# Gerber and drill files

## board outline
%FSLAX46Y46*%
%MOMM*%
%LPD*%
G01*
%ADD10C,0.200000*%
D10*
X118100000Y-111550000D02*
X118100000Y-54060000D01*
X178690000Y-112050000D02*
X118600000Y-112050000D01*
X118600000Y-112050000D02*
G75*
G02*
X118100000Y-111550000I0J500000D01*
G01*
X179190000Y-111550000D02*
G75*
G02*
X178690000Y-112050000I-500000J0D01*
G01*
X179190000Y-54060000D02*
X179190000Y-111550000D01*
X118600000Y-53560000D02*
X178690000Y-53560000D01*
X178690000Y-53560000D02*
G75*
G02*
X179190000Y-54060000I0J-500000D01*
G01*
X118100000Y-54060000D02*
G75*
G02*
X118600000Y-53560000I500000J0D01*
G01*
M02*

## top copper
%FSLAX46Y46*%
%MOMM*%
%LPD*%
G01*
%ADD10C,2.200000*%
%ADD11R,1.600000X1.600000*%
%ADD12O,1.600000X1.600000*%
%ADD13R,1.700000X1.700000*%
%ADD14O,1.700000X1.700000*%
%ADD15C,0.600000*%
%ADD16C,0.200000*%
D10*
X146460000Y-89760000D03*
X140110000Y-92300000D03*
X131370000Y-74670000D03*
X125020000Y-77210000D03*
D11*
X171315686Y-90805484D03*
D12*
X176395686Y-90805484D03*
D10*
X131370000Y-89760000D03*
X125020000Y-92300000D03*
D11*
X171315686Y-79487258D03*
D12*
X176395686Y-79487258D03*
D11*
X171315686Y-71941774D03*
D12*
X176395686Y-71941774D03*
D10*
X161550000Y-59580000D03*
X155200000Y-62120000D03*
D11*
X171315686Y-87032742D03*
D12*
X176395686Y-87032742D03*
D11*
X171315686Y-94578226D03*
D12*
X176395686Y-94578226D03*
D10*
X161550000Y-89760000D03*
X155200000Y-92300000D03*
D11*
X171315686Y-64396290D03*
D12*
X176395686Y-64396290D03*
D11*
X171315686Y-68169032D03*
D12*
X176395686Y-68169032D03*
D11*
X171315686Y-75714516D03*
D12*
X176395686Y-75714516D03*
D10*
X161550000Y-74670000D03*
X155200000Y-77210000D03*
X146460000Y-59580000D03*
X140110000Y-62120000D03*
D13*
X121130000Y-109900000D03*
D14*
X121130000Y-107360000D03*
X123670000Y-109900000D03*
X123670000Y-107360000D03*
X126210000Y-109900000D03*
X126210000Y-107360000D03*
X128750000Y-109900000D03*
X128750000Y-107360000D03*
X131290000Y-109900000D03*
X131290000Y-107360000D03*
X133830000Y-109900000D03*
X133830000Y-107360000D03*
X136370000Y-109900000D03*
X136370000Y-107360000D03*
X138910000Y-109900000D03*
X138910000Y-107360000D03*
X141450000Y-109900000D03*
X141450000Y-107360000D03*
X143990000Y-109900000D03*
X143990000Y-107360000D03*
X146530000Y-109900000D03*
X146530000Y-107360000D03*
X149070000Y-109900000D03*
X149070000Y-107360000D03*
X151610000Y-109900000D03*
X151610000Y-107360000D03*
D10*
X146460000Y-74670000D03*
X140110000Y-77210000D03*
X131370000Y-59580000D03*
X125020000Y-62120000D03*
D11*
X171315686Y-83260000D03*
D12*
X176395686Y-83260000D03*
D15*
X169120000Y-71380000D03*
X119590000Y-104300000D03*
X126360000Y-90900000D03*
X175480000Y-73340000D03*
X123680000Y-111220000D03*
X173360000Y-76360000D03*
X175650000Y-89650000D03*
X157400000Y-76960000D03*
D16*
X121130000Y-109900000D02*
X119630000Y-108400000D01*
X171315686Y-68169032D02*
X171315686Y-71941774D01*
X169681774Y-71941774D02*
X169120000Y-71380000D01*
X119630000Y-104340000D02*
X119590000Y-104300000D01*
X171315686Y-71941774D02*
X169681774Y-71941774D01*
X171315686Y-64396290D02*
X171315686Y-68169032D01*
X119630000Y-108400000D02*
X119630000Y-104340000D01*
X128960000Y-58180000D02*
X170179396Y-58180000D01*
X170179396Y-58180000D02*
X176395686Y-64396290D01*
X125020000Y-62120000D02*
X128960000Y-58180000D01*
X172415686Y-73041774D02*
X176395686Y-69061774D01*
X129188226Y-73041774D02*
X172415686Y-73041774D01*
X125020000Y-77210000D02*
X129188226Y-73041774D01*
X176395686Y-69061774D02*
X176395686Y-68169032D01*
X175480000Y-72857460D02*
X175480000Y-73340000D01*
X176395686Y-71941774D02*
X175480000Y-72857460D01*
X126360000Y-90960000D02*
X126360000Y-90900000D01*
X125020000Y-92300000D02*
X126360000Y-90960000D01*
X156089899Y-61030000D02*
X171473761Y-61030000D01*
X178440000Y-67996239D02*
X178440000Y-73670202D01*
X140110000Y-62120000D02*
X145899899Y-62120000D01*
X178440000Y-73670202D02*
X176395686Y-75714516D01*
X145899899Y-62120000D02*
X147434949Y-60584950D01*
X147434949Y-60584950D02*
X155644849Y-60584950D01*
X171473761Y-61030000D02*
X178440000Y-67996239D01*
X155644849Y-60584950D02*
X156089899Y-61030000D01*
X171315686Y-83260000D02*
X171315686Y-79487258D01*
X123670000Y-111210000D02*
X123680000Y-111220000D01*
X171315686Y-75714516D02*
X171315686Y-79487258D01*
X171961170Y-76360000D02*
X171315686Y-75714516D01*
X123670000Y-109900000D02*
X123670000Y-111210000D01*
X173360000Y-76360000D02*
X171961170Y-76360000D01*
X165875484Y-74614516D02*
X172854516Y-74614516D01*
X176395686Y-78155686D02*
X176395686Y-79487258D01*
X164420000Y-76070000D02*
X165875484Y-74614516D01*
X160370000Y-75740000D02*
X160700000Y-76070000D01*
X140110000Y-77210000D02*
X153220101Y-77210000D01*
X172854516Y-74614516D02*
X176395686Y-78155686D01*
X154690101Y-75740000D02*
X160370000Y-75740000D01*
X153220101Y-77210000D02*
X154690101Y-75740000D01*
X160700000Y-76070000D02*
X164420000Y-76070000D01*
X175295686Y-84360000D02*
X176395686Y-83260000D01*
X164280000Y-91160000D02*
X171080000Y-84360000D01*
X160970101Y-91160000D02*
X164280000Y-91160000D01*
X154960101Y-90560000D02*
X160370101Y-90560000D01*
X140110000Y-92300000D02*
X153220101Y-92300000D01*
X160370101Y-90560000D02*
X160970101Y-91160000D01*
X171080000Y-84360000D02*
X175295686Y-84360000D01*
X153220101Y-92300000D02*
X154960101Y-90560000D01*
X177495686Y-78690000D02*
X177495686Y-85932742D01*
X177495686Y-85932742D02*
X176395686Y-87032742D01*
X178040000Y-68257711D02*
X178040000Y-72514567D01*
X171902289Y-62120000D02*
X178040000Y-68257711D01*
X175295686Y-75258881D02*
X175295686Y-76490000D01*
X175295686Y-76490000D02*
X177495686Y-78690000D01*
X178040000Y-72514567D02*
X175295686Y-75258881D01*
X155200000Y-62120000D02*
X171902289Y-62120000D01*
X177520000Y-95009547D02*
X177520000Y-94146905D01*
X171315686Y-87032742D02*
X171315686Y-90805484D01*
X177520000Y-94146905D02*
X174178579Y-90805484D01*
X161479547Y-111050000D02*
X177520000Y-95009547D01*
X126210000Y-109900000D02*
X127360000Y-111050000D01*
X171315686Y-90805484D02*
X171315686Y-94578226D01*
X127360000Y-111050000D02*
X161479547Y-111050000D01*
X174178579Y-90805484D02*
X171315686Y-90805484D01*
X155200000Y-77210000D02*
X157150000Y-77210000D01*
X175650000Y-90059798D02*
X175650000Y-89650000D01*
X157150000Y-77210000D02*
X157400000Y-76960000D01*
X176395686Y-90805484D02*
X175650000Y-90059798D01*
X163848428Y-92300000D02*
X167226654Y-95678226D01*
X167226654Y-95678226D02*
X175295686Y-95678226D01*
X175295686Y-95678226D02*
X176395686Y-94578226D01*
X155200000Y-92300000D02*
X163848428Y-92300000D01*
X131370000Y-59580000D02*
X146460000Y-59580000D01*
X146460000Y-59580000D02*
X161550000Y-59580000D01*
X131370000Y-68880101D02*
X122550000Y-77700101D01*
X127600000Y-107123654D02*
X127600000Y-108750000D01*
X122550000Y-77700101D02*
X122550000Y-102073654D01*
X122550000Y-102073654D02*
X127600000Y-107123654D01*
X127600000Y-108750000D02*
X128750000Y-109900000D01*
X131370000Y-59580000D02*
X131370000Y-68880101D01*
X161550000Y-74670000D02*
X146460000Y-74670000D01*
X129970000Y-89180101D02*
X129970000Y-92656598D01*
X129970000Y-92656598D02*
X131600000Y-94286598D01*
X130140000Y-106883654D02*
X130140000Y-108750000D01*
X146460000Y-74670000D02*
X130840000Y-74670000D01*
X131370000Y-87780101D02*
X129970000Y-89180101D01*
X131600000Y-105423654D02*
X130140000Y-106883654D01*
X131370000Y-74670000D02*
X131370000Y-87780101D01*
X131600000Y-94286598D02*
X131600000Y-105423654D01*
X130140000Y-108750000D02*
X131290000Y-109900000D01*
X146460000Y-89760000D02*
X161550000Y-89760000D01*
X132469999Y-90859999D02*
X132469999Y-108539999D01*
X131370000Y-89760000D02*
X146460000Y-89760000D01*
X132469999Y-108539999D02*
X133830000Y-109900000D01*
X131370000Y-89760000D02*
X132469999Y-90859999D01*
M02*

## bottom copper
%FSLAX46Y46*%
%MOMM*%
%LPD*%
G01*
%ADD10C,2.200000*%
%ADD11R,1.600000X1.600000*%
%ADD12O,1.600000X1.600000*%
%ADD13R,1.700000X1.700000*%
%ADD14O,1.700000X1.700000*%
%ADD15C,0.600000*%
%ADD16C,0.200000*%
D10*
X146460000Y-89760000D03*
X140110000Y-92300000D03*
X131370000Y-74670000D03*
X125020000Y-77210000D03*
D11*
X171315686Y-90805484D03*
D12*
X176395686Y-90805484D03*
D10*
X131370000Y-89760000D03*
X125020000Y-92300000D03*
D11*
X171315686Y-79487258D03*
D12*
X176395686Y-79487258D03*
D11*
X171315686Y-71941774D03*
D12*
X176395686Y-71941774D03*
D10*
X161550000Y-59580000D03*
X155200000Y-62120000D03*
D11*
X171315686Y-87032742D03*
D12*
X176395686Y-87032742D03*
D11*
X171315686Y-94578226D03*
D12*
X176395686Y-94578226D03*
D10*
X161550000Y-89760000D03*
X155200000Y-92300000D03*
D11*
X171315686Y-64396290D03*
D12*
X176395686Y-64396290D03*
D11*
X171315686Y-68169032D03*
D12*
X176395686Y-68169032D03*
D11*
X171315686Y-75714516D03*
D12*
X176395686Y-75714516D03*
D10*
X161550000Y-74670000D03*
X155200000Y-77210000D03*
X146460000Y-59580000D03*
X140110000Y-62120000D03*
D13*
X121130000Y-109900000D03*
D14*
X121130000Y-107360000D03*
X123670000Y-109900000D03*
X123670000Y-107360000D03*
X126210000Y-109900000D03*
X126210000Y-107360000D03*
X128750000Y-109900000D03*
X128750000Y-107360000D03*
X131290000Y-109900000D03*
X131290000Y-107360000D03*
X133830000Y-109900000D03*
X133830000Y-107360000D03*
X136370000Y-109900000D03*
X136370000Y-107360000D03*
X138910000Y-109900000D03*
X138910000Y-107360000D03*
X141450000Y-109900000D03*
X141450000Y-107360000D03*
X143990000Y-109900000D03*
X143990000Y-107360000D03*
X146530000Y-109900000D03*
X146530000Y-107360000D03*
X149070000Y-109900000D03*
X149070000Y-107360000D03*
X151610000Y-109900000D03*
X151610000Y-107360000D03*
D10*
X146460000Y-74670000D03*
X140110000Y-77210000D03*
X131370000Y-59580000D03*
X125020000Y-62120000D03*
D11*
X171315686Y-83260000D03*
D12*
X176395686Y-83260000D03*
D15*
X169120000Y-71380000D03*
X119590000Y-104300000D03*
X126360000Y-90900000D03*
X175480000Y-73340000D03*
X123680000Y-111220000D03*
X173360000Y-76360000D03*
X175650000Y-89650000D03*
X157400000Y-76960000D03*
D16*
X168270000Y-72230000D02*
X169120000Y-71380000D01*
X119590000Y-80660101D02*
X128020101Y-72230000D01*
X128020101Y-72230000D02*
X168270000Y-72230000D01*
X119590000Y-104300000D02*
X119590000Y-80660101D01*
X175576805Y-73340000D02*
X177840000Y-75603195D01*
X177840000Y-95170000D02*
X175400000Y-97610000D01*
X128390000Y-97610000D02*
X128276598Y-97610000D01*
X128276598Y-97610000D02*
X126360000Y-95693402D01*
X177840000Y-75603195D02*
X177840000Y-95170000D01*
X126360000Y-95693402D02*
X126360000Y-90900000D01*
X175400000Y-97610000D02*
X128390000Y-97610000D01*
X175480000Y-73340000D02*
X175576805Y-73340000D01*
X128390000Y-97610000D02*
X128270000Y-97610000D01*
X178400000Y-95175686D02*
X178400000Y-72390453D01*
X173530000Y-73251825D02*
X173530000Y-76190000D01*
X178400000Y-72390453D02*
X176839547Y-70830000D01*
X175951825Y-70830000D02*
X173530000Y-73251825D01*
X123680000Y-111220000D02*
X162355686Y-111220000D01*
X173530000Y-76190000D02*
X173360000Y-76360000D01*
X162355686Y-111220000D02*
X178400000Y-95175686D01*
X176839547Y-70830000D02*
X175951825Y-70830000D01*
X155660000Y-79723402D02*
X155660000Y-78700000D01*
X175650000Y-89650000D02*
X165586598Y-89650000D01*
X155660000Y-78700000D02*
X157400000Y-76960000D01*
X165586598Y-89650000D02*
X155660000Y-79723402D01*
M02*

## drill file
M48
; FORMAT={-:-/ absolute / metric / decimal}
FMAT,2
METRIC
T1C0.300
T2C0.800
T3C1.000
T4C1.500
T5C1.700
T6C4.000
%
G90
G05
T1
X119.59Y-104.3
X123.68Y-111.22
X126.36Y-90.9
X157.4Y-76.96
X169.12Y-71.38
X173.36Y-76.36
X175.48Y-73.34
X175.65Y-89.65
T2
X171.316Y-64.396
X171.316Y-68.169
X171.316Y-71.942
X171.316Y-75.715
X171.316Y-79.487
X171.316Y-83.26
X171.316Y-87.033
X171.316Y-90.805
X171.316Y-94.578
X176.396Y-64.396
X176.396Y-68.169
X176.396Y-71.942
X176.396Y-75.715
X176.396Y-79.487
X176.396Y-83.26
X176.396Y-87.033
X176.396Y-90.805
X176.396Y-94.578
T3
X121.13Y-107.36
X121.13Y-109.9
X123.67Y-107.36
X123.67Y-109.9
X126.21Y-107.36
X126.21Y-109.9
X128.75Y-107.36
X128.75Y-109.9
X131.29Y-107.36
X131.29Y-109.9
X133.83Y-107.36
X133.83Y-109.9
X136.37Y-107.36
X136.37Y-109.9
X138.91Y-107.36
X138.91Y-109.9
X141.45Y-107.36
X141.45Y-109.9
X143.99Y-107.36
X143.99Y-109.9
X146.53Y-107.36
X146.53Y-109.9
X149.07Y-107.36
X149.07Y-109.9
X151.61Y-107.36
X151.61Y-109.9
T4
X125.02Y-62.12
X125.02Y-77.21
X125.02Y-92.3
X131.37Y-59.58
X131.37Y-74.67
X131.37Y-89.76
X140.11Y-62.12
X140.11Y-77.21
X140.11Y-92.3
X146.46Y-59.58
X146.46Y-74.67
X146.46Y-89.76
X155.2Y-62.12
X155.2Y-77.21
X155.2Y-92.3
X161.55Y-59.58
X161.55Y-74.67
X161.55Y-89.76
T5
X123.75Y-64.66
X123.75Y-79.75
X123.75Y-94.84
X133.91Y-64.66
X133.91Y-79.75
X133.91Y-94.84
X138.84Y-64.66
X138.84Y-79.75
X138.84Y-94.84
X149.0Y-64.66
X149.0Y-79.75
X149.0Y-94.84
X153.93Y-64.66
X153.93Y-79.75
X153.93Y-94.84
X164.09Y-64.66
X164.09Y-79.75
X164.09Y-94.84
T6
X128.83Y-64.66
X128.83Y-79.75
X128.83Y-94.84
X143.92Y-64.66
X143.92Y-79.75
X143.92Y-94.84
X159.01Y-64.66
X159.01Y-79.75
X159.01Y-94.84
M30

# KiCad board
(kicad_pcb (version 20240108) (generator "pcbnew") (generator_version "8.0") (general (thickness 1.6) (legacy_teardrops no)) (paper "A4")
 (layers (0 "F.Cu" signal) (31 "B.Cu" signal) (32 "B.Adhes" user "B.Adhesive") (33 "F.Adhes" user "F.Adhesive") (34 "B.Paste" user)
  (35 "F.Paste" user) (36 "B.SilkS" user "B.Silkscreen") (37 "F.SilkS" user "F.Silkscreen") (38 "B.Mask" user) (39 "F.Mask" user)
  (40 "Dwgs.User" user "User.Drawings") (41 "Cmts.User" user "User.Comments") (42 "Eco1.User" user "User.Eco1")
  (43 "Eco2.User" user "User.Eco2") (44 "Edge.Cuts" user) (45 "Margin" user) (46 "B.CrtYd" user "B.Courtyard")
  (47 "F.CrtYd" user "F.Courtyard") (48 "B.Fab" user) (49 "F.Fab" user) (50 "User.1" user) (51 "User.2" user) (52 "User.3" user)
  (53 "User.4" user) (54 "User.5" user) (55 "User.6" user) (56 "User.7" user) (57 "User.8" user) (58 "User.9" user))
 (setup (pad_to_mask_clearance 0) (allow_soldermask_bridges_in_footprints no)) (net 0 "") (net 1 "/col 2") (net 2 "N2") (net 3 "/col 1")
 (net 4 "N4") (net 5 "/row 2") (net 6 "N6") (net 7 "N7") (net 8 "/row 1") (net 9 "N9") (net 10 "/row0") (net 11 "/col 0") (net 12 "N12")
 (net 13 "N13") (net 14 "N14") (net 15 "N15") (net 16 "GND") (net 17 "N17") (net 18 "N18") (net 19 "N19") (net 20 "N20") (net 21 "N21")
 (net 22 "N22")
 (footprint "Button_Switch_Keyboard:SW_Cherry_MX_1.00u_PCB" (layer "F.Cu") (at 146.46 89.76)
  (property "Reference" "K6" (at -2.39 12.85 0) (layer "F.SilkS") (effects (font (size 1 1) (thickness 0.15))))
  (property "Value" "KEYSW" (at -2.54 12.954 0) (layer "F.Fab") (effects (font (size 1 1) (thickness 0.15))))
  (pad "" np_thru_hole circle (at -7.62 5.08) (size 1.7 1.7) (drill 1.7) (layers "*.Cu" "*.Mask"))
  (pad "" np_thru_hole circle (at -2.54 5.08) (size 4 4) (drill 4) (layers "*.Cu" "*.Mask"))
  (pad "" np_thru_hole circle (at 2.54 5.08) (size 1.7 1.7) (drill 1.7) (layers "*.Cu" "*.Mask"))
  (pad "1" thru_hole circle (at 0 0) (size 2.2 2.2) (drill 1.5) (layers "*.Cu" "*.Mask") (remove_unused_layers no) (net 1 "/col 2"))
  (pad "2" thru_hole circle (at -6.35 2.54) (size 2.2 2.2) (drill 1.5) (layers "*.Cu" "*.Mask") (remove_unused_layers no) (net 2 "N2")))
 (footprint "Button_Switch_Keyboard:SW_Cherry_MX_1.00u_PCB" (layer "F.Cu") (at 131.37 74.67)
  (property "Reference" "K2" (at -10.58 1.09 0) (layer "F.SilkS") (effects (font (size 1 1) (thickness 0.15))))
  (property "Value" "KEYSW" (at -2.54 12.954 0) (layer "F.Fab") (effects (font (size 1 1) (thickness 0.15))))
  (pad "" np_thru_hole circle (at -7.62 5.08) (size 1.7 1.7) (drill 1.7) (layers "*.Cu" "*.Mask"))
  (pad "" np_thru_hole circle (at -2.54 5.08) (size 4 4) (drill 4) (layers "*.Cu" "*.Mask"))
  (pad "" np_thru_hole circle (at 2.54 5.08) (size 1.7 1.7) (drill 1.7) (layers "*.Cu" "*.Mask"))
  (pad "1" thru_hole circle (at 0 0) (size 2.2 2.2) (drill 1.5) (layers "*.Cu" "*.Mask") (remove_unused_layers no) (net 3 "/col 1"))
  (pad "2" thru_hole circle (at -6.35 2.54) (size 2.2 2.2) (drill 1.5) (layers "*.Cu" "*.Mask") (remove_unused_layers no) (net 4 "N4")))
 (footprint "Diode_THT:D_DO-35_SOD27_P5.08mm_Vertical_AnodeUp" (layer "F.Cu") (at 171.315686 90.805484)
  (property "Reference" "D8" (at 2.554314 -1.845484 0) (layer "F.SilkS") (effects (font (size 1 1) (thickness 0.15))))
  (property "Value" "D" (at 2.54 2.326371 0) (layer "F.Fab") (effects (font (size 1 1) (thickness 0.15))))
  (pad "1" thru_hole rect (at 0 0) (size 1.6 1.6) (drill 0.8) (layers "*.Cu" "*.Mask") (remove_unused_layers no) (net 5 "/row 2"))
  (pad "2" thru_hole oval (at 5.08 0) (size 1.6 1.6) (drill 0.8) (layers "*.Cu" "*.Mask") (remove_unused_layers no) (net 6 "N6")))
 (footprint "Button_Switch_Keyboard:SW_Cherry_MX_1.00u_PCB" (layer "F.Cu") (at 131.37 89.76)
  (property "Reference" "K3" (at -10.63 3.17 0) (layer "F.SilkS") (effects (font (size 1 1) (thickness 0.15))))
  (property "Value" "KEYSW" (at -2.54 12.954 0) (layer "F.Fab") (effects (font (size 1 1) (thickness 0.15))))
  (pad "" np_thru_hole circle (at -7.62 5.08) (size 1.7 1.7) (drill 1.7) (layers "*.Cu" "*.Mask"))
  (pad "" np_thru_hole circle (at -2.54 5.08) (size 4 4) (drill 4) (layers "*.Cu" "*.Mask"))
  (pad "" np_thru_hole circle (at 2.54 5.08) (size 1.7 1.7) (drill 1.7) (layers "*.Cu" "*.Mask"))
  (pad "1" thru_hole circle (at 0 0) (size 2.2 2.2) (drill 1.5) (layers "*.Cu" "*.Mask") (remove_unused_layers no) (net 1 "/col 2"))
  (pad "2" thru_hole circle (at -6.35 2.54) (size 2.2 2.2) (drill 1.5) (layers "*.Cu" "*.Mask") (remove_unused_layers no) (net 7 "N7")))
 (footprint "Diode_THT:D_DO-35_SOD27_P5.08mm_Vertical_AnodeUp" (layer "F.Cu") (at 171.315686 79.487258)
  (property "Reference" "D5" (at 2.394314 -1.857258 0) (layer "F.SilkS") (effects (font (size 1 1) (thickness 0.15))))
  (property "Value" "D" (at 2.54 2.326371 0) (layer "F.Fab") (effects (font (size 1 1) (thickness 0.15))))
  (pad "1" thru_hole rect (at 0 0) (size 1.6 1.6) (drill 0.8) (layers "*.Cu" "*.Mask") (remove_unused_layers no) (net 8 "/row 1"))
  (pad "2" thru_hole oval (at 5.08 0) (size 1.6 1.6) (drill 0.8) (layers "*.Cu" "*.Mask") (remove_unused_layers no) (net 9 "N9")))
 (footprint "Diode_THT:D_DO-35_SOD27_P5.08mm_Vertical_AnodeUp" (layer "F.Cu") (at 171.315686 71.941774)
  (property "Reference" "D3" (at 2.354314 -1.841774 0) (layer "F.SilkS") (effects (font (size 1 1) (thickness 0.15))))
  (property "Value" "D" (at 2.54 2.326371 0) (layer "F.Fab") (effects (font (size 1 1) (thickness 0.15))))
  (pad "1" thru_hole rect (at 0 0) (size 1.6 1.6) (drill 0.8) (layers "*.Cu" "*.Mask") (remove_unused_layers no) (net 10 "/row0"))
  (pad "2" thru_hole oval (at 5.08 0) (size 1.6 1.6) (drill 0.8) (layers "*.Cu" "*.Mask") (remove_unused_layers no) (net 7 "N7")))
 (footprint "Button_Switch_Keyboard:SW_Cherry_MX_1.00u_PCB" (layer "F.Cu") (at 161.55 59.58)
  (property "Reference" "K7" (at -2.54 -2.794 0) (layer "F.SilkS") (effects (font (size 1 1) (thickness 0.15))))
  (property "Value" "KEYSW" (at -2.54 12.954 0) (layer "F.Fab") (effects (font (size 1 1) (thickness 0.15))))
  (pad "" np_thru_hole circle (at -7.62 5.08) (size 1.7 1.7) (drill 1.7) (layers "*.Cu" "*.Mask"))
  (pad "" np_thru_hole circle (at -2.54 5.08) (size 4 4) (drill 4) (layers "*.Cu" "*.Mask"))
  (pad "" np_thru_hole circle (at 2.54 5.08) (size 1.7 1.7) (drill 1.7) (layers "*.Cu" "*.Mask"))
  (pad "1" thru_hole circle (at 0 0) (size 2.2 2.2) (drill 1.5) (layers "*.Cu" "*.Mask") (remove_unused_layers no) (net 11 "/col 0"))
  (pad "2" thru_hole circle (at -6.35 2.54) (size 2.2 2.2) (drill 1.5) (layers "*.Cu" "*.Mask") (remove_unused_layers no) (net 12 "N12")))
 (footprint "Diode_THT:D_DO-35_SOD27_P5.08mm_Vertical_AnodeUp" (layer "F.Cu") (at 171.315686 87.032742)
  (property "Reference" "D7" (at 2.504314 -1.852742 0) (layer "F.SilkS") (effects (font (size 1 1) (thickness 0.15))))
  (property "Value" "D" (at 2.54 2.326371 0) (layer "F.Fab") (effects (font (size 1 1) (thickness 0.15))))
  (pad "1" thru_hole rect (at 0 0) (size 1.6 1.6) (drill 0.8) (layers "*.Cu" "*.Mask") (remove_unused_layers no) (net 5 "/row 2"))
  (pad "2" thru_hole oval (at 5.08 0) (size 1.6 1.6) (drill 0.8) (layers "*.Cu" "*.Mask") (remove_unused_layers no) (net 12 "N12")))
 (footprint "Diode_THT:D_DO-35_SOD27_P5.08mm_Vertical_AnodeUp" (layer "F.Cu") (at 171.315686 94.578226)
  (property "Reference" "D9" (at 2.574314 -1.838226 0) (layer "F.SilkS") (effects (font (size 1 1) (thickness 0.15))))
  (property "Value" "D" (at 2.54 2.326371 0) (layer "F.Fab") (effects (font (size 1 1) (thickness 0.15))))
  (pad "1" thru_hole rect (at 0 0) (size 1.6 1.6) (drill 0.8) (layers "*.Cu" "*.Mask") (remove_unused_layers no) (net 5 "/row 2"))
  (pad "2" thru_hole oval (at 5.08 0) (size 1.6 1.6) (drill 0.8) (layers "*.Cu" "*.Mask") (remove_unused_layers no) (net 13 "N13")))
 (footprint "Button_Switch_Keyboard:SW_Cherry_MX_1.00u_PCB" (layer "F.Cu") (at 161.55 89.76)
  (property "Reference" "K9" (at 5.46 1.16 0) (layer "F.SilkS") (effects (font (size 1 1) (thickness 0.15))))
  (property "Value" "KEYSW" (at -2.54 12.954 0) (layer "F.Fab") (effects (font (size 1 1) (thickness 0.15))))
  (pad "" np_thru_hole circle (at -7.62 5.08) (size 1.7 1.7) (drill 1.7) (layers "*.Cu" "*.Mask"))
  (pad "" np_thru_hole circle (at -2.54 5.08) (size 4 4) (drill 4) (layers "*.Cu" "*.Mask"))
  (pad "" np_thru_hole circle (at 2.54 5.08) (size 1.7 1.7) (drill 1.7) (layers "*.Cu" "*.Mask"))
  (pad "1" thru_hole circle (at 0 0) (size 2.2 2.2) (drill 1.5) (layers "*.Cu" "*.Mask") (remove_unused_layers no) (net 1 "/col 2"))
  (pad "2" thru_hole circle (at -6.35 2.54) (size 2.2 2.2) (drill 1.5) (layers "*.Cu" "*.Mask") (remove_unused_layers no) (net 13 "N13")))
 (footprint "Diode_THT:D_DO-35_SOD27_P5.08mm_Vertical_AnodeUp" (layer "F.Cu") (at 171.315686 64.39629)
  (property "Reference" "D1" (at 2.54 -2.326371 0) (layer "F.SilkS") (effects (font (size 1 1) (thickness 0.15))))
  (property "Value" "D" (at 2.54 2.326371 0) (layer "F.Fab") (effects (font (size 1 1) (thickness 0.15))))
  (pad "1" thru_hole rect (at 0 0) (size 1.6 1.6) (drill 0.8) (layers "*.Cu" "*.Mask") (remove_unused_layers no) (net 10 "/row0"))
  (pad "2" thru_hole oval (at 5.08 0) (size 1.6 1.6) (drill 0.8) (layers "*.Cu" "*.Mask") (remove_unused_layers no) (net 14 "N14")))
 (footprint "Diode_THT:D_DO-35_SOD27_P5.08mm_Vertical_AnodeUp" (layer "F.Cu") (at 171.315686 68.169032)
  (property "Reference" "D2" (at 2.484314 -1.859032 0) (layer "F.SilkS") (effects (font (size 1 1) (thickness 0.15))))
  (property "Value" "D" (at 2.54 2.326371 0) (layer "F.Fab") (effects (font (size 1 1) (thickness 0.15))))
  (pad "1" thru_hole rect (at 0 0) (size 1.6 1.6) (drill 0.8) (layers "*.Cu" "*.Mask") (remove_unused_layers no) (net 10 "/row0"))
  (pad "2" thru_hole oval (at 5.08 0) (size 1.6 1.6) (drill 0.8) (layers "*.Cu" "*.Mask") (remove_unused_layers no) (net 4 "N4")))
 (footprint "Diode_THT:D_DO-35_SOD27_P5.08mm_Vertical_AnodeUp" (layer "F.Cu") (at 171.315686 75.714516)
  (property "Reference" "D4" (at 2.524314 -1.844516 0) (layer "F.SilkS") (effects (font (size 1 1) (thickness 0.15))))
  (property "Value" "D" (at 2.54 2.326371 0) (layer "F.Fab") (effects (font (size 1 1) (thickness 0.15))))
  (pad "1" thru_hole rect (at 0 0) (size 1.6 1.6) (drill 0.8) (layers "*.Cu" "*.Mask") (remove_unused_layers no) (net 8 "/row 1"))
  (pad "2" thru_hole oval (at 5.08 0) (size 1.6 1.6) (drill 0.8) (layers "*.Cu" "*.Mask") (remove_unused_layers no) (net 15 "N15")))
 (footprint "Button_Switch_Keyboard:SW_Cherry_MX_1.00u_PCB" (layer "F.Cu") (at 161.55 74.67)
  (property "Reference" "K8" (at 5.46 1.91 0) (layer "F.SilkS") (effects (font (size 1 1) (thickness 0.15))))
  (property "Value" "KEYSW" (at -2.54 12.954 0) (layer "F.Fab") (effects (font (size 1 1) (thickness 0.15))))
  (pad "" np_thru_hole circle (at -7.62 5.08) (size 1.7 1.7) (drill 1.7) (layers "*.Cu" "*.Mask"))
  (pad "" np_thru_hole circle (at -2.54 5.08) (size 4 4) (drill 4) (layers "*.Cu" "*.Mask"))
  (pad "" np_thru_hole circle (at 2.54 5.08) (size 1.7 1.7) (drill 1.7) (layers "*.Cu" "*.Mask"))
  (pad "1" thru_hole circle (at 0 0) (size 2.2 2.2) (drill 1.5) (layers "*.Cu" "*.Mask") (remove_unused_layers no) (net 3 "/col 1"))
  (pad "2" thru_hole circle (at -6.35 2.54) (size 2.2 2.2) (drill 1.5) (layers "*.Cu" "*.Mask") (remove_unused_layers no) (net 6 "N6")))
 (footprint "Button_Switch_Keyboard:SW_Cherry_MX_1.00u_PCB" (layer "F.Cu") (at 146.46 59.58)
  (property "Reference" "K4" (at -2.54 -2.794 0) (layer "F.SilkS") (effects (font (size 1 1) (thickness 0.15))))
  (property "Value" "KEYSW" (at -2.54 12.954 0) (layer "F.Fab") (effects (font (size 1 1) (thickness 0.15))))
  (pad "" np_thru_hole circle (at -7.62 5.08) (size 1.7 1.7) (drill 1.7) (layers "*.Cu" "*.Mask"))
  (pad "" np_thru_hole circle (at -2.54 5.08) (size 4 4) (drill 4) (layers "*.Cu" "*.Mask"))
  (pad "" np_thru_hole circle (at 2.54 5.08) (size 1.7 1.7) (drill 1.7) (layers "*.Cu" "*.Mask"))
  (pad "1" thru_hole circle (at 0 0) (size 2.2 2.2) (drill 1.5) (layers "*.Cu" "*.Mask") (remove_unused_layers no) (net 11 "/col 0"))
  (pad "2" thru_hole circle (at -6.35 2.54) (size 2.2 2.2) (drill 1.5) (layers "*.Cu" "*.Mask") (remove_unused_layers no) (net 15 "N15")))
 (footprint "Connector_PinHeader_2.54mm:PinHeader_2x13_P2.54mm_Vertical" (layer "F.Cu") (at 121.13 109.9 90)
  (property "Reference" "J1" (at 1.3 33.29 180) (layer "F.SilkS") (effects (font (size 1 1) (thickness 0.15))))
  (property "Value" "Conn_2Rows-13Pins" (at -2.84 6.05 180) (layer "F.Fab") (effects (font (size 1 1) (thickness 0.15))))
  (pad "1" thru_hole rect (at 0 0 90) (size 1.7 1.7) (drill 1) (layers "*.Cu" "*.Mask") (remove_unused_layers no) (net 10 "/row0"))
  (pad "2" thru_hole oval (at 2.54 0 90) (size 1.7 1.7) (drill 1) (layers "*.Cu" "*.Mask") (remove_unused_layers no) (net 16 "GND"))
  (pad "3" thru_hole oval (at 0 2.54 90) (size 1.7 1.7) (drill 1) (layers "*.Cu" "*.Mask") (remove_unused_layers no) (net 8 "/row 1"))
  (pad "4" thru_hole oval (at 2.54 2.54 90) (size 1.7 1.7) (drill 1) (layers "*.Cu" "*.Mask") (remove_unused_layers no) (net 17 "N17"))
  (pad "5" thru_hole oval (at 0 5.08 90) (size 1.7 1.7) (drill 1) (layers "*.Cu" "*.Mask") (remove_unused_layers no) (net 5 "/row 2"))
  (pad "6" thru_hole oval (at 2.54 5.08 90) (size 1.7 1.7) (drill 1) (layers "*.Cu" "*.Mask") (remove_unused_layers no) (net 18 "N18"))
  (pad "7" thru_hole oval (at 0 7.62 90) (size 1.7 1.7) (drill 1) (layers "*.Cu" "*.Mask") (remove_unused_layers no) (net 11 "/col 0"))
  (pad "8" thru_hole oval (at 2.54 7.62 90) (size 1.7 1.7) (drill 1) (layers "*.Cu" "*.Mask") (remove_unused_layers no) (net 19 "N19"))
  (pad "9" thru_hole oval (at 0 10.16 90) (size 1.7 1.7) (drill 1) (layers "*.Cu" "*.Mask") (remove_unused_layers no) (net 3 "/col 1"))
  (pad "10" thru_hole oval (at 2.54 10.16 90) (size 1.7 1.7) (drill 1) (layers "*.Cu" "*.Mask") (remove_unused_layers no) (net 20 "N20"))
  (pad "11" thru_hole oval (at 0 12.7 90) (size 1.7 1.7) (drill 1) (layers "*.Cu" "*.Mask") (remove_unused_layers no) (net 1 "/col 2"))
  (pad "12" thru_hole oval (at 2.54 12.7 90) (size 1.7 1.7) (drill 1) (layers "*.Cu" "*.Mask") (remove_unused_layers no) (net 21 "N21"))
  (pad "13" thru_hole oval (at 0 15.24 90) (size 1.7 1.7) (drill 1) (layers "*.Cu" "*.Mask") (remove_unused_layers no) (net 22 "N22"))
  (pad "14" thru_hole oval (at 2.54 15.24 90) (size 1.7 1.7) (drill 1) (layers "*.Cu" "*.Mask") (remove_unused_layers no))
  (pad "15" thru_hole oval (at 0 17.78 90) (size 1.7 1.7) (drill 1) (layers "*.Cu" "*.Mask") (remove_unused_layers no))
  (pad "16" thru_hole oval (at 2.54 17.78 90) (size 1.7 1.7) (drill 1) (layers "*.Cu" "*.Mask") (remove_unused_layers no))
  (pad "17" thru_hole oval (at 0 20.32 90) (size 1.7 1.7) (drill 1) (layers "*.Cu" "*.Mask") (remove_unused_layers no))
  (pad "18" thru_hole oval (at 2.54 20.32 90) (size 1.7 1.7) (drill 1) (layers "*.Cu" "*.Mask") (remove_unused_layers no))
  (pad "19" thru_hole oval (at 0 22.86 90) (size 1.7 1.7) (drill 1) (layers "*.Cu" "*.Mask") (remove_unused_layers no))
  (pad "20" thru_hole oval (at 2.54 22.86 90) (size 1.7 1.7) (drill 1) (layers "*.Cu" "*.Mask") (remove_unused_layers no))
  (pad "21" thru_hole oval (at 0 25.4 90) (size 1.7 1.7) (drill 1) (layers "*.Cu" "*.Mask") (remove_unused_layers no))
  (pad "22" thru_hole oval (at 2.54 25.4 90) (size 1.7 1.7) (drill 1) (layers "*.Cu" "*.Mask") (remove_unused_layers no))
  (pad "23" thru_hole oval (at 0 27.94 90) (size 1.7 1.7) (drill 1) (layers "*.Cu" "*.Mask") (remove_unused_layers no))
  (pad "24" thru_hole oval (at 2.54 27.94 90) (size 1.7 1.7) (drill 1) (layers "*.Cu" "*.Mask") (remove_unused_layers no))
  (pad "25" thru_hole oval (at 0 30.48 90) (size 1.7 1.7) (drill 1) (layers "*.Cu" "*.Mask") (remove_unused_layers no))
  (pad "26" thru_hole oval (at 2.54 30.48 90) (size 1.7 1.7) (drill 1) (layers "*.Cu" "*.Mask") (remove_unused_layers no)))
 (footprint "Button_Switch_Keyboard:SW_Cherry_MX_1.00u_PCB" (layer "F.Cu") (at 146.46 74.67)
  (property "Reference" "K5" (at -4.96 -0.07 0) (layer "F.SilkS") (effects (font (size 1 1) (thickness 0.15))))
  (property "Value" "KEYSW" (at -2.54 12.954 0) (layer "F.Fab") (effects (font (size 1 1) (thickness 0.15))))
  (pad "" np_thru_hole circle (at -7.62 5.08) (size 1.7 1.7) (drill 1.7) (layers "*.Cu" "*.Mask"))
  (pad "" np_thru_hole circle (at -2.54 5.08) (size 4 4) (drill 4) (layers "*.Cu" "*.Mask"))
  (pad "" np_thru_hole circle (at 2.54 5.08) (size 1.7 1.7) (drill 1.7) (layers "*.Cu" "*.Mask"))
  (pad "1" thru_hole circle (at 0 0) (size 2.2 2.2) (drill 1.5) (layers "*.Cu" "*.Mask") (remove_unused_layers no) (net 3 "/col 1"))
  (pad "2" thru_hole circle (at -6.35 2.54) (size 2.2 2.2) (drill 1.5) (layers "*.Cu" "*.Mask") (remove_unused_layers no) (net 9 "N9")))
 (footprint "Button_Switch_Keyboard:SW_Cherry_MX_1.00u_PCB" (layer "F.Cu") (at 131.37 59.58)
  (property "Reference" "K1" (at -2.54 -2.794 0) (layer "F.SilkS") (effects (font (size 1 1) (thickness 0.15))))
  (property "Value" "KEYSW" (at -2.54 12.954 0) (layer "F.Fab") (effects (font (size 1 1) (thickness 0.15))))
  (pad "" np_thru_hole circle (at -7.62 5.08) (size 1.7 1.7) (drill 1.7) (layers "*.Cu" "*.Mask"))
  (pad "" np_thru_hole circle (at -2.54 5.08) (size 4 4) (drill 4) (layers "*.Cu" "*.Mask"))
  (pad "" np_thru_hole circle (at 2.54 5.08) (size 1.7 1.7) (drill 1.7) (layers "*.Cu" "*.Mask"))
  (pad "1" thru_hole circle (at 0 0) (size 2.2 2.2) (drill 1.5) (layers "*.Cu" "*.Mask") (remove_unused_layers no) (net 11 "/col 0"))
  (pad "2" thru_hole circle (at -6.35 2.54) (size 2.2 2.2) (drill 1.5) (layers "*.Cu" "*.Mask") (remove_unused_layers no) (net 14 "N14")))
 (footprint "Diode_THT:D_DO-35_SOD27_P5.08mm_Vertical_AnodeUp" (layer "F.Cu") (at 171.315686 83.26)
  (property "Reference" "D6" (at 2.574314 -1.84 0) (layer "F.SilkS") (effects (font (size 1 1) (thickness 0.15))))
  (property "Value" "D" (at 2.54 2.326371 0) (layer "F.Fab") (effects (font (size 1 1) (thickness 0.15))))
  (pad "1" thru_hole rect (at 0 0) (size 1.6 1.6) (drill 0.8) (layers "*.Cu" "*.Mask") (remove_unused_layers no) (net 8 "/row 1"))
  (pad "2" thru_hole oval (at 5.08 0) (size 1.6 1.6) (drill 0.8) (layers "*.Cu" "*.Mask") (remove_unused_layers no) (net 2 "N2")))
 (gr_line (start 118.1 111.55) (end 118.1 54.06) (stroke (width 0.2) (type default)) (layer "Edge.Cuts"))
 (gr_line (start 178.69 112.05) (end 118.6 112.05) (stroke (width 0.2) (type default)) (layer "Edge.Cuts"))
 (gr_arc (start 118.6 112.05) (mid 118.246447 111.903553) (end 118.1 111.55) (stroke (width 0.2) (type default)) (layer "Edge.Cuts"))
 (gr_arc (start 179.19 111.55) (mid 179.043553 111.903553) (end 178.69 112.05) (stroke (width 0.2) (type default)) (layer "Edge.Cuts"))
 (gr_line (start 179.19 54.06) (end 179.19 111.55) (stroke (width 0.2) (type default)) (layer "Edge.Cuts"))
 (gr_line (start 118.6 53.56) (end 178.69 53.56) (stroke (width 0.2) (type default)) (layer "Edge.Cuts"))
 (gr_arc (start 178.69 53.56) (mid 179.043553 53.706447) (end 179.19 54.06) (stroke (width 0.2) (type default)) (layer "Edge.Cuts"))
 (gr_arc (start 118.1 54.06) (mid 118.246447 53.706447) (end 118.6 53.56) (stroke (width 0.2) (type default)) (layer "Edge.Cuts"))
 (segment (start 121.13 109.9) (end 119.63 108.4) (width 0.2) (layer "F.Cu") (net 10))
 (segment (start 171.315686 68.169032) (end 171.315686 71.941774) (width 0.2) (layer "F.Cu") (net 10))
 (segment (start 169.681774 71.941774) (end 169.12 71.38) (width 0.2) (layer "F.Cu") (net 10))
 (segment (start 119.63 104.34) (end 119.59 104.3) (width 0.2) (layer "F.Cu") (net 10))
 (segment (start 171.315686 71.941774) (end 169.681774 71.941774) (width 0.2) (layer "F.Cu") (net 10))
 (segment (start 171.315686 64.39629) (end 171.315686 68.169032) (width 0.2) (layer "F.Cu") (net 10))
 (segment (start 119.63 108.4) (end 119.63 104.34) (width 0.2) (layer "F.Cu") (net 10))
 (via (at 169.12 71.38) (size 0.6) (drill 0.3) (layers "F.Cu" "B.Cu") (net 10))
 (via (at 119.59 104.3) (size 0.6) (drill 0.3) (layers "F.Cu" "B.Cu") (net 10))
 (segment (start 168.27 72.23) (end 169.12 71.38) (width 0.2) (layer "B.Cu") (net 10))
 (segment (start 119.59 80.660101) (end 128.020101 72.23) (width 0.2) (layer "B.Cu") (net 10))
 (segment (start 128.020101 72.23) (end 168.27 72.23) (width 0.2) (layer "B.Cu") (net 10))
 (segment (start 119.59 104.3) (end 119.59 80.660101) (width 0.2) (layer "B.Cu") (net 10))
 (segment (start 128.96 58.18) (end 170.179396 58.18) (width 0.2) (layer "F.Cu") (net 14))
 (segment (start 170.179396 58.18) (end 176.395686 64.39629) (width 0.2) (layer "F.Cu") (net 14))
 (segment (start 125.02 62.12) (end 128.96 58.18) (width 0.2) (layer "F.Cu") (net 14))
 (segment (start 172.415686 73.041774) (end 176.395686 69.061774) (width 0.2) (layer "F.Cu") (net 4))
 (segment (start 129.188226 73.041774) (end 172.415686 73.041774) (width 0.2) (layer "F.Cu") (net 4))
 (segment (start 125.02 77.21) (end 129.188226 73.041774) (width 0.2) (layer "F.Cu") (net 4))
 (segment (start 176.395686 69.061774) (end 176.395686 68.169032) (width 0.2) (layer "F.Cu") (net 4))
 (segment (start 175.48 72.85746) (end 175.48 73.34) (width 0.2) (layer "F.Cu") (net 7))
 (segment (start 176.395686 71.941774) (end 175.48 72.85746) (width 0.2) (layer "F.Cu") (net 7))
 (segment (start 126.36 90.96) (end 126.36 90.9) (width 0.2) (layer "F.Cu") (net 7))
 (segment (start 125.02 92.3) (end 126.36 90.96) (width 0.2) (layer "F.Cu") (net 7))
 (via (at 126.36 90.9) (size 0.6) (drill 0.3) (layers "F.Cu" "B.Cu") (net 7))
 (via (at 175.48 73.34) (size 0.6) (drill 0.3) (layers "F.Cu" "B.Cu") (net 7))
 (segment (start 175.576805 73.34) (end 177.84 75.603195) (width 0.2) (layer "B.Cu") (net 7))
 (segment (start 177.84 95.17) (end 175.4 97.61) (width 0.2) (layer "B.Cu") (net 7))
 (segment (start 128.39 97.61) (end 128.276598 97.61) (width 0.2) (layer "B.Cu") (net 7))
 (segment (start 128.276598 97.61) (end 126.36 95.693402) (width 0.2) (layer "B.Cu") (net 7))
 (segment (start 177.84 75.603195) (end 177.84 95.17) (width 0.2) (layer "B.Cu") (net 7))
 (segment (start 126.36 95.693402) (end 126.36 90.9) (width 0.2) (layer "B.Cu") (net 7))
 (segment (start 175.4 97.61) (end 128.39 97.61) (width 0.2) (layer "B.Cu") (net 7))
 (segment (start 175.48 73.34) (end 175.576805 73.34) (width 0.2) (layer "B.Cu") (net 7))
 (segment (start 128.39 97.61) (end 128.27 97.61) (width 0.2) (layer "B.Cu") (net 7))
 (segment (start 156.089899 61.03) (end 171.473761 61.03) (width 0.2) (layer "F.Cu") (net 15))
 (segment (start 178.44 67.996239) (end 178.44 73.670202) (width 0.2) (layer "F.Cu") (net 15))
 (segment (start 140.11 62.12) (end 145.899899 62.12) (width 0.2) (layer "F.Cu") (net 15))
 (segment (start 178.44 73.670202) (end 176.395686 75.714516) (width 0.2) (layer "F.Cu") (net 15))
 (segment (start 145.899899 62.12) (end 147.434949 60.58495) (width 0.2) (layer "F.Cu") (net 15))
 (segment (start 147.434949 60.58495) (end 155.644849 60.58495) (width 0.2) (layer "F.Cu") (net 15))
 (segment (start 171.473761 61.03) (end 178.44 67.996239) (width 0.2) (layer "F.Cu") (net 15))
 (segment (start 155.644849 60.58495) (end 156.089899 61.03) (width 0.2) (layer "F.Cu") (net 15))
 (segment (start 171.315686 83.26) (end 171.315686 79.487258) (width 0.2) (layer "F.Cu") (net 8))
 (segment (start 123.67 111.21) (end 123.68 111.22) (width 0.2) (layer "F.Cu") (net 8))
 (segment (start 171.315686 75.714516) (end 171.315686 79.487258) (width 0.2) (layer "F.Cu") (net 8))
 (segment (start 171.96117 76.36) (end 171.315686 75.714516) (width 0.2) (layer "F.Cu") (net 8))
 (segment (start 123.67 109.9) (end 123.67 111.21) (width 0.2) (layer "F.Cu") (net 8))
 (segment (start 173.36 76.36) (end 171.96117 76.36) (width 0.2) (layer "F.Cu") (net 8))
 (via (at 123.68 111.22) (size 0.6) (drill 0.3) (layers "F.Cu" "B.Cu") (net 8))
 (via (at 173.36 76.36) (size 0.6) (drill 0.3) (layers "F.Cu" "B.Cu") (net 8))
 (segment (start 178.4 95.175686) (end 178.4 72.390453) (width 0.2) (layer "B.Cu") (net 8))
 (segment (start 173.53 73.251825) (end 173.53 76.19) (width 0.2) (layer "B.Cu") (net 8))
 (segment (start 178.4 72.390453) (end 176.839547 70.83) (width 0.2) (layer "B.Cu") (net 8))
 (segment (start 175.951825 70.83) (end 173.53 73.251825) (width 0.2) (layer "B.Cu") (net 8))
 (segment (start 123.68 111.22) (end 162.355686 111.22) (width 0.2) (layer "B.Cu") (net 8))
 (segment (start 173.53 76.19) (end 173.36 76.36) (width 0.2) (layer "B.Cu") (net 8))
 (segment (start 162.355686 111.22) (end 178.4 95.175686) (width 0.2) (layer "B.Cu") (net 8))
 (segment (start 176.839547 70.83) (end 175.951825 70.83) (width 0.2) (layer "B.Cu") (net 8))
 (segment (start 165.875484 74.614516) (end 172.854516 74.614516) (width 0.2) (layer "F.Cu") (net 9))
 (segment (start 176.395686 78.155686) (end 176.395686 79.487258) (width 0.2) (layer "F.Cu") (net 9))
 (segment (start 164.42 76.07) (end 165.875484 74.614516) (width 0.2) (layer "F.Cu") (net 9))
 (segment (start 160.37 75.74) (end 160.7 76.07) (width 0.2) (layer "F.Cu") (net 9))
 (segment (start 140.11 77.21) (end 153.220101 77.21) (width 0.2) (layer "F.Cu") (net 9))
 (segment (start 172.854516 74.614516) (end 176.395686 78.155686) (width 0.2) (layer "F.Cu") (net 9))
 (segment (start 154.690101 75.74) (end 160.37 75.74) (width 0.2) (layer "F.Cu") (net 9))
 (segment (start 153.220101 77.21) (end 154.690101 75.74) (width 0.2) (layer "F.Cu") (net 9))
 (segment (start 160.7 76.07) (end 164.42 76.07) (width 0.2) (layer "F.Cu") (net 9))
 (segment (start 175.295686 84.36) (end 176.395686 83.26) (width 0.2) (layer "F.Cu") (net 2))
 (segment (start 164.28 91.16) (end 171.08 84.36) (width 0.2) (layer "F.Cu") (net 2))
 (segment (start 160.970101 91.16) (end 164.28 91.16) (width 0.2) (layer "F.Cu") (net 2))
 (segment (start 154.960101 90.56) (end 160.370101 90.56) (width 0.2) (layer "F.Cu") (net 2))
 (segment (start 140.11 92.3) (end 153.220101 92.3) (width 0.2) (layer "F.Cu") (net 2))
 (segment (start 160.370101 90.56) (end 160.970101 91.16) (width 0.2) (layer "F.Cu") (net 2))
 (segment (start 171.08 84.36) (end 175.295686 84.36) (width 0.2) (layer "F.Cu") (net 2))
 (segment (start 153.220101 92.3) (end 154.960101 90.56) (width 0.2) (layer "F.Cu") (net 2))
 (segment (start 177.495686 78.69) (end 177.495686 85.932742) (width 0.2) (layer "F.Cu") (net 12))
 (segment (start 177.495686 85.932742) (end 176.395686 87.032742) (width 0.2) (layer "F.Cu") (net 12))
 (segment (start 178.04 68.257711) (end 178.04 72.514567) (width 0.2) (layer "F.Cu") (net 12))
 (segment (start 171.902289 62.12) (end 178.04 68.257711) (width 0.2) (layer "F.Cu") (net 12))
 (segment (start 175.295686 75.258881) (end 175.295686 76.49) (width 0.2) (layer "F.Cu") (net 12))
 (segment (start 175.295686 76.49) (end 177.495686 78.69) (width 0.2) (layer "F.Cu") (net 12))
 (segment (start 178.04 72.514567) (end 175.295686 75.258881) (width 0.2) (layer "F.Cu") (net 12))
 (segment (start 155.2 62.12) (end 171.902289 62.12) (width 0.2) (layer "F.Cu") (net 12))
 (segment (start 177.52 95.009547) (end 177.52 94.146905) (width 0.2) (layer "F.Cu") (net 5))
 (segment (start 171.315686 87.032742) (end 171.315686 90.805484) (width 0.2) (layer "F.Cu") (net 5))
 (segment (start 177.52 94.146905) (end 174.178579 90.805484) (width 0.2) (layer "F.Cu") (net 5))
 (segment (start 161.479547 111.05) (end 177.52 95.009547) (width 0.2) (layer "F.Cu") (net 5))
 (segment (start 126.21 109.9) (end 127.36 111.05) (width 0.2) (layer "F.Cu") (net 5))
 (segment (start 171.315686 90.805484) (end 171.315686 94.578226) (width 0.2) (layer "F.Cu") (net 5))
 (segment (start 127.36 111.05) (end 161.479547 111.05) (width 0.2) (layer "F.Cu") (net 5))
 (segment (start 174.178579 90.805484) (end 171.315686 90.805484) (width 0.2) (layer "F.Cu") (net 5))
 (segment (start 155.2 77.21) (end 157.15 77.21) (width 0.2) (layer "F.Cu") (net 6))
 (segment (start 175.65 90.059798) (end 175.65 89.65) (width 0.2) (layer "F.Cu") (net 6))
 (segment (start 157.15 77.21) (end 157.4 76.96) (width 0.2) (layer "F.Cu") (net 6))
 (segment (start 176.395686 90.805484) (end 175.65 90.059798) (width 0.2) (layer "F.Cu") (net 6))
 (via (at 175.65 89.65) (size 0.6) (drill 0.3) (layers "F.Cu" "B.Cu") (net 6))
 (via (at 157.4 76.96) (size 0.6) (drill 0.3) (layers "F.Cu" "B.Cu") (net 6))
 (segment (start 155.66 79.723402) (end 155.66 78.7) (width 0.2) (layer "B.Cu") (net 6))
 (segment (start 175.65 89.65) (end 165.586598 89.65) (width 0.2) (layer "B.Cu") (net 6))
 (segment (start 155.66 78.7) (end 157.4 76.96) (width 0.2) (layer "B.Cu") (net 6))
 (segment (start 165.586598 89.65) (end 155.66 79.723402) (width 0.2) (layer "B.Cu") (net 6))
 (segment (start 163.848428 92.3) (end 167.226654 95.678226) (width 0.2) (layer "F.Cu") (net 13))
 (segment (start 167.226654 95.678226) (end 175.295686 95.678226) (width 0.2) (layer "F.Cu") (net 13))
 (segment (start 175.295686 95.678226) (end 176.395686 94.578226) (width 0.2) (layer "F.Cu") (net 13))
 (segment (start 155.2 92.3) (end 163.848428 92.3) (width 0.2) (layer "F.Cu") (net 13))
 (segment (start 131.37 59.58) (end 146.46 59.58) (width 0.2) (layer "F.Cu") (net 11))
 (segment (start 146.46 59.58) (end 161.55 59.58) (width 0.2) (layer "F.Cu") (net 11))
 (segment (start 131.37 68.880101) (end 122.55 77.700101) (width 0.2) (layer "F.Cu") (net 11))
 (segment (start 127.6 107.123654) (end 127.6 108.75) (width 0.2) (layer "F.Cu") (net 11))
 (segment (start 122.55 77.700101) (end 122.55 102.073654) (width 0.2) (layer "F.Cu") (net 11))
 (segment (start 122.55 102.073654) (end 127.6 107.123654) (width 0.2) (layer "F.Cu") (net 11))
 (segment (start 127.6 108.75) (end 128.75 109.9) (width 0.2) (layer "F.Cu") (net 11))
 (segment (start 131.37 59.58) (end 131.37 68.880101) (width 0.2) (layer "F.Cu") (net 11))
 (segment (start 161.55 74.67) (end 146.46 74.67) (width 0.2) (layer "F.Cu") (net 3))
 (segment (start 129.97 89.180101) (end 129.97 92.656598) (width 0.2) (layer "F.Cu") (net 3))
 (segment (start 129.97 92.656598) (end 131.6 94.286598) (width 0.2) (layer "F.Cu") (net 3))
 (segment (start 130.14 106.883654) (end 130.14 108.75) (width 0.2) (layer "F.Cu") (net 3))
 (segment (start 146.46 74.67) (end 130.84 74.67) (width 0.2) (layer "F.Cu") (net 3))
 (segment (start 131.37 87.780101) (end 129.97 89.180101) (width 0.2) (layer "F.Cu") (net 3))
 (segment (start 131.6 105.423654) (end 130.14 106.883654) (width 0.2) (layer "F.Cu") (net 3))
 (segment (start 131.37 74.67) (end 131.37 87.780101) (width 0.2) (layer "F.Cu") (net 3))
 (segment (start 131.6 94.286598) (end 131.6 105.423654) (width 0.2) (layer "F.Cu") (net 3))
 (segment (start 130.14 108.75) (end 131.29 109.9) (width 0.2) (layer "F.Cu") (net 3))
 (segment (start 146.46 89.76) (end 161.55 89.76) (width 0.2) (layer "F.Cu") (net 1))
 (segment (start 132.469999 90.859999) (end 132.469999 108.539999) (width 0.2) (layer "F.Cu") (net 1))
 (segment (start 131.37 89.76) (end 146.46 89.76) (width 0.2) (layer "F.Cu") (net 1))
 (segment (start 132.469999 108.539999) (end 133.83 109.9) (width 0.2) (layer "F.Cu") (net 1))
 (segment (start 131.37 89.76) (end 132.469999 90.859999) (width 0.2) (layer "F.Cu") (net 1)))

